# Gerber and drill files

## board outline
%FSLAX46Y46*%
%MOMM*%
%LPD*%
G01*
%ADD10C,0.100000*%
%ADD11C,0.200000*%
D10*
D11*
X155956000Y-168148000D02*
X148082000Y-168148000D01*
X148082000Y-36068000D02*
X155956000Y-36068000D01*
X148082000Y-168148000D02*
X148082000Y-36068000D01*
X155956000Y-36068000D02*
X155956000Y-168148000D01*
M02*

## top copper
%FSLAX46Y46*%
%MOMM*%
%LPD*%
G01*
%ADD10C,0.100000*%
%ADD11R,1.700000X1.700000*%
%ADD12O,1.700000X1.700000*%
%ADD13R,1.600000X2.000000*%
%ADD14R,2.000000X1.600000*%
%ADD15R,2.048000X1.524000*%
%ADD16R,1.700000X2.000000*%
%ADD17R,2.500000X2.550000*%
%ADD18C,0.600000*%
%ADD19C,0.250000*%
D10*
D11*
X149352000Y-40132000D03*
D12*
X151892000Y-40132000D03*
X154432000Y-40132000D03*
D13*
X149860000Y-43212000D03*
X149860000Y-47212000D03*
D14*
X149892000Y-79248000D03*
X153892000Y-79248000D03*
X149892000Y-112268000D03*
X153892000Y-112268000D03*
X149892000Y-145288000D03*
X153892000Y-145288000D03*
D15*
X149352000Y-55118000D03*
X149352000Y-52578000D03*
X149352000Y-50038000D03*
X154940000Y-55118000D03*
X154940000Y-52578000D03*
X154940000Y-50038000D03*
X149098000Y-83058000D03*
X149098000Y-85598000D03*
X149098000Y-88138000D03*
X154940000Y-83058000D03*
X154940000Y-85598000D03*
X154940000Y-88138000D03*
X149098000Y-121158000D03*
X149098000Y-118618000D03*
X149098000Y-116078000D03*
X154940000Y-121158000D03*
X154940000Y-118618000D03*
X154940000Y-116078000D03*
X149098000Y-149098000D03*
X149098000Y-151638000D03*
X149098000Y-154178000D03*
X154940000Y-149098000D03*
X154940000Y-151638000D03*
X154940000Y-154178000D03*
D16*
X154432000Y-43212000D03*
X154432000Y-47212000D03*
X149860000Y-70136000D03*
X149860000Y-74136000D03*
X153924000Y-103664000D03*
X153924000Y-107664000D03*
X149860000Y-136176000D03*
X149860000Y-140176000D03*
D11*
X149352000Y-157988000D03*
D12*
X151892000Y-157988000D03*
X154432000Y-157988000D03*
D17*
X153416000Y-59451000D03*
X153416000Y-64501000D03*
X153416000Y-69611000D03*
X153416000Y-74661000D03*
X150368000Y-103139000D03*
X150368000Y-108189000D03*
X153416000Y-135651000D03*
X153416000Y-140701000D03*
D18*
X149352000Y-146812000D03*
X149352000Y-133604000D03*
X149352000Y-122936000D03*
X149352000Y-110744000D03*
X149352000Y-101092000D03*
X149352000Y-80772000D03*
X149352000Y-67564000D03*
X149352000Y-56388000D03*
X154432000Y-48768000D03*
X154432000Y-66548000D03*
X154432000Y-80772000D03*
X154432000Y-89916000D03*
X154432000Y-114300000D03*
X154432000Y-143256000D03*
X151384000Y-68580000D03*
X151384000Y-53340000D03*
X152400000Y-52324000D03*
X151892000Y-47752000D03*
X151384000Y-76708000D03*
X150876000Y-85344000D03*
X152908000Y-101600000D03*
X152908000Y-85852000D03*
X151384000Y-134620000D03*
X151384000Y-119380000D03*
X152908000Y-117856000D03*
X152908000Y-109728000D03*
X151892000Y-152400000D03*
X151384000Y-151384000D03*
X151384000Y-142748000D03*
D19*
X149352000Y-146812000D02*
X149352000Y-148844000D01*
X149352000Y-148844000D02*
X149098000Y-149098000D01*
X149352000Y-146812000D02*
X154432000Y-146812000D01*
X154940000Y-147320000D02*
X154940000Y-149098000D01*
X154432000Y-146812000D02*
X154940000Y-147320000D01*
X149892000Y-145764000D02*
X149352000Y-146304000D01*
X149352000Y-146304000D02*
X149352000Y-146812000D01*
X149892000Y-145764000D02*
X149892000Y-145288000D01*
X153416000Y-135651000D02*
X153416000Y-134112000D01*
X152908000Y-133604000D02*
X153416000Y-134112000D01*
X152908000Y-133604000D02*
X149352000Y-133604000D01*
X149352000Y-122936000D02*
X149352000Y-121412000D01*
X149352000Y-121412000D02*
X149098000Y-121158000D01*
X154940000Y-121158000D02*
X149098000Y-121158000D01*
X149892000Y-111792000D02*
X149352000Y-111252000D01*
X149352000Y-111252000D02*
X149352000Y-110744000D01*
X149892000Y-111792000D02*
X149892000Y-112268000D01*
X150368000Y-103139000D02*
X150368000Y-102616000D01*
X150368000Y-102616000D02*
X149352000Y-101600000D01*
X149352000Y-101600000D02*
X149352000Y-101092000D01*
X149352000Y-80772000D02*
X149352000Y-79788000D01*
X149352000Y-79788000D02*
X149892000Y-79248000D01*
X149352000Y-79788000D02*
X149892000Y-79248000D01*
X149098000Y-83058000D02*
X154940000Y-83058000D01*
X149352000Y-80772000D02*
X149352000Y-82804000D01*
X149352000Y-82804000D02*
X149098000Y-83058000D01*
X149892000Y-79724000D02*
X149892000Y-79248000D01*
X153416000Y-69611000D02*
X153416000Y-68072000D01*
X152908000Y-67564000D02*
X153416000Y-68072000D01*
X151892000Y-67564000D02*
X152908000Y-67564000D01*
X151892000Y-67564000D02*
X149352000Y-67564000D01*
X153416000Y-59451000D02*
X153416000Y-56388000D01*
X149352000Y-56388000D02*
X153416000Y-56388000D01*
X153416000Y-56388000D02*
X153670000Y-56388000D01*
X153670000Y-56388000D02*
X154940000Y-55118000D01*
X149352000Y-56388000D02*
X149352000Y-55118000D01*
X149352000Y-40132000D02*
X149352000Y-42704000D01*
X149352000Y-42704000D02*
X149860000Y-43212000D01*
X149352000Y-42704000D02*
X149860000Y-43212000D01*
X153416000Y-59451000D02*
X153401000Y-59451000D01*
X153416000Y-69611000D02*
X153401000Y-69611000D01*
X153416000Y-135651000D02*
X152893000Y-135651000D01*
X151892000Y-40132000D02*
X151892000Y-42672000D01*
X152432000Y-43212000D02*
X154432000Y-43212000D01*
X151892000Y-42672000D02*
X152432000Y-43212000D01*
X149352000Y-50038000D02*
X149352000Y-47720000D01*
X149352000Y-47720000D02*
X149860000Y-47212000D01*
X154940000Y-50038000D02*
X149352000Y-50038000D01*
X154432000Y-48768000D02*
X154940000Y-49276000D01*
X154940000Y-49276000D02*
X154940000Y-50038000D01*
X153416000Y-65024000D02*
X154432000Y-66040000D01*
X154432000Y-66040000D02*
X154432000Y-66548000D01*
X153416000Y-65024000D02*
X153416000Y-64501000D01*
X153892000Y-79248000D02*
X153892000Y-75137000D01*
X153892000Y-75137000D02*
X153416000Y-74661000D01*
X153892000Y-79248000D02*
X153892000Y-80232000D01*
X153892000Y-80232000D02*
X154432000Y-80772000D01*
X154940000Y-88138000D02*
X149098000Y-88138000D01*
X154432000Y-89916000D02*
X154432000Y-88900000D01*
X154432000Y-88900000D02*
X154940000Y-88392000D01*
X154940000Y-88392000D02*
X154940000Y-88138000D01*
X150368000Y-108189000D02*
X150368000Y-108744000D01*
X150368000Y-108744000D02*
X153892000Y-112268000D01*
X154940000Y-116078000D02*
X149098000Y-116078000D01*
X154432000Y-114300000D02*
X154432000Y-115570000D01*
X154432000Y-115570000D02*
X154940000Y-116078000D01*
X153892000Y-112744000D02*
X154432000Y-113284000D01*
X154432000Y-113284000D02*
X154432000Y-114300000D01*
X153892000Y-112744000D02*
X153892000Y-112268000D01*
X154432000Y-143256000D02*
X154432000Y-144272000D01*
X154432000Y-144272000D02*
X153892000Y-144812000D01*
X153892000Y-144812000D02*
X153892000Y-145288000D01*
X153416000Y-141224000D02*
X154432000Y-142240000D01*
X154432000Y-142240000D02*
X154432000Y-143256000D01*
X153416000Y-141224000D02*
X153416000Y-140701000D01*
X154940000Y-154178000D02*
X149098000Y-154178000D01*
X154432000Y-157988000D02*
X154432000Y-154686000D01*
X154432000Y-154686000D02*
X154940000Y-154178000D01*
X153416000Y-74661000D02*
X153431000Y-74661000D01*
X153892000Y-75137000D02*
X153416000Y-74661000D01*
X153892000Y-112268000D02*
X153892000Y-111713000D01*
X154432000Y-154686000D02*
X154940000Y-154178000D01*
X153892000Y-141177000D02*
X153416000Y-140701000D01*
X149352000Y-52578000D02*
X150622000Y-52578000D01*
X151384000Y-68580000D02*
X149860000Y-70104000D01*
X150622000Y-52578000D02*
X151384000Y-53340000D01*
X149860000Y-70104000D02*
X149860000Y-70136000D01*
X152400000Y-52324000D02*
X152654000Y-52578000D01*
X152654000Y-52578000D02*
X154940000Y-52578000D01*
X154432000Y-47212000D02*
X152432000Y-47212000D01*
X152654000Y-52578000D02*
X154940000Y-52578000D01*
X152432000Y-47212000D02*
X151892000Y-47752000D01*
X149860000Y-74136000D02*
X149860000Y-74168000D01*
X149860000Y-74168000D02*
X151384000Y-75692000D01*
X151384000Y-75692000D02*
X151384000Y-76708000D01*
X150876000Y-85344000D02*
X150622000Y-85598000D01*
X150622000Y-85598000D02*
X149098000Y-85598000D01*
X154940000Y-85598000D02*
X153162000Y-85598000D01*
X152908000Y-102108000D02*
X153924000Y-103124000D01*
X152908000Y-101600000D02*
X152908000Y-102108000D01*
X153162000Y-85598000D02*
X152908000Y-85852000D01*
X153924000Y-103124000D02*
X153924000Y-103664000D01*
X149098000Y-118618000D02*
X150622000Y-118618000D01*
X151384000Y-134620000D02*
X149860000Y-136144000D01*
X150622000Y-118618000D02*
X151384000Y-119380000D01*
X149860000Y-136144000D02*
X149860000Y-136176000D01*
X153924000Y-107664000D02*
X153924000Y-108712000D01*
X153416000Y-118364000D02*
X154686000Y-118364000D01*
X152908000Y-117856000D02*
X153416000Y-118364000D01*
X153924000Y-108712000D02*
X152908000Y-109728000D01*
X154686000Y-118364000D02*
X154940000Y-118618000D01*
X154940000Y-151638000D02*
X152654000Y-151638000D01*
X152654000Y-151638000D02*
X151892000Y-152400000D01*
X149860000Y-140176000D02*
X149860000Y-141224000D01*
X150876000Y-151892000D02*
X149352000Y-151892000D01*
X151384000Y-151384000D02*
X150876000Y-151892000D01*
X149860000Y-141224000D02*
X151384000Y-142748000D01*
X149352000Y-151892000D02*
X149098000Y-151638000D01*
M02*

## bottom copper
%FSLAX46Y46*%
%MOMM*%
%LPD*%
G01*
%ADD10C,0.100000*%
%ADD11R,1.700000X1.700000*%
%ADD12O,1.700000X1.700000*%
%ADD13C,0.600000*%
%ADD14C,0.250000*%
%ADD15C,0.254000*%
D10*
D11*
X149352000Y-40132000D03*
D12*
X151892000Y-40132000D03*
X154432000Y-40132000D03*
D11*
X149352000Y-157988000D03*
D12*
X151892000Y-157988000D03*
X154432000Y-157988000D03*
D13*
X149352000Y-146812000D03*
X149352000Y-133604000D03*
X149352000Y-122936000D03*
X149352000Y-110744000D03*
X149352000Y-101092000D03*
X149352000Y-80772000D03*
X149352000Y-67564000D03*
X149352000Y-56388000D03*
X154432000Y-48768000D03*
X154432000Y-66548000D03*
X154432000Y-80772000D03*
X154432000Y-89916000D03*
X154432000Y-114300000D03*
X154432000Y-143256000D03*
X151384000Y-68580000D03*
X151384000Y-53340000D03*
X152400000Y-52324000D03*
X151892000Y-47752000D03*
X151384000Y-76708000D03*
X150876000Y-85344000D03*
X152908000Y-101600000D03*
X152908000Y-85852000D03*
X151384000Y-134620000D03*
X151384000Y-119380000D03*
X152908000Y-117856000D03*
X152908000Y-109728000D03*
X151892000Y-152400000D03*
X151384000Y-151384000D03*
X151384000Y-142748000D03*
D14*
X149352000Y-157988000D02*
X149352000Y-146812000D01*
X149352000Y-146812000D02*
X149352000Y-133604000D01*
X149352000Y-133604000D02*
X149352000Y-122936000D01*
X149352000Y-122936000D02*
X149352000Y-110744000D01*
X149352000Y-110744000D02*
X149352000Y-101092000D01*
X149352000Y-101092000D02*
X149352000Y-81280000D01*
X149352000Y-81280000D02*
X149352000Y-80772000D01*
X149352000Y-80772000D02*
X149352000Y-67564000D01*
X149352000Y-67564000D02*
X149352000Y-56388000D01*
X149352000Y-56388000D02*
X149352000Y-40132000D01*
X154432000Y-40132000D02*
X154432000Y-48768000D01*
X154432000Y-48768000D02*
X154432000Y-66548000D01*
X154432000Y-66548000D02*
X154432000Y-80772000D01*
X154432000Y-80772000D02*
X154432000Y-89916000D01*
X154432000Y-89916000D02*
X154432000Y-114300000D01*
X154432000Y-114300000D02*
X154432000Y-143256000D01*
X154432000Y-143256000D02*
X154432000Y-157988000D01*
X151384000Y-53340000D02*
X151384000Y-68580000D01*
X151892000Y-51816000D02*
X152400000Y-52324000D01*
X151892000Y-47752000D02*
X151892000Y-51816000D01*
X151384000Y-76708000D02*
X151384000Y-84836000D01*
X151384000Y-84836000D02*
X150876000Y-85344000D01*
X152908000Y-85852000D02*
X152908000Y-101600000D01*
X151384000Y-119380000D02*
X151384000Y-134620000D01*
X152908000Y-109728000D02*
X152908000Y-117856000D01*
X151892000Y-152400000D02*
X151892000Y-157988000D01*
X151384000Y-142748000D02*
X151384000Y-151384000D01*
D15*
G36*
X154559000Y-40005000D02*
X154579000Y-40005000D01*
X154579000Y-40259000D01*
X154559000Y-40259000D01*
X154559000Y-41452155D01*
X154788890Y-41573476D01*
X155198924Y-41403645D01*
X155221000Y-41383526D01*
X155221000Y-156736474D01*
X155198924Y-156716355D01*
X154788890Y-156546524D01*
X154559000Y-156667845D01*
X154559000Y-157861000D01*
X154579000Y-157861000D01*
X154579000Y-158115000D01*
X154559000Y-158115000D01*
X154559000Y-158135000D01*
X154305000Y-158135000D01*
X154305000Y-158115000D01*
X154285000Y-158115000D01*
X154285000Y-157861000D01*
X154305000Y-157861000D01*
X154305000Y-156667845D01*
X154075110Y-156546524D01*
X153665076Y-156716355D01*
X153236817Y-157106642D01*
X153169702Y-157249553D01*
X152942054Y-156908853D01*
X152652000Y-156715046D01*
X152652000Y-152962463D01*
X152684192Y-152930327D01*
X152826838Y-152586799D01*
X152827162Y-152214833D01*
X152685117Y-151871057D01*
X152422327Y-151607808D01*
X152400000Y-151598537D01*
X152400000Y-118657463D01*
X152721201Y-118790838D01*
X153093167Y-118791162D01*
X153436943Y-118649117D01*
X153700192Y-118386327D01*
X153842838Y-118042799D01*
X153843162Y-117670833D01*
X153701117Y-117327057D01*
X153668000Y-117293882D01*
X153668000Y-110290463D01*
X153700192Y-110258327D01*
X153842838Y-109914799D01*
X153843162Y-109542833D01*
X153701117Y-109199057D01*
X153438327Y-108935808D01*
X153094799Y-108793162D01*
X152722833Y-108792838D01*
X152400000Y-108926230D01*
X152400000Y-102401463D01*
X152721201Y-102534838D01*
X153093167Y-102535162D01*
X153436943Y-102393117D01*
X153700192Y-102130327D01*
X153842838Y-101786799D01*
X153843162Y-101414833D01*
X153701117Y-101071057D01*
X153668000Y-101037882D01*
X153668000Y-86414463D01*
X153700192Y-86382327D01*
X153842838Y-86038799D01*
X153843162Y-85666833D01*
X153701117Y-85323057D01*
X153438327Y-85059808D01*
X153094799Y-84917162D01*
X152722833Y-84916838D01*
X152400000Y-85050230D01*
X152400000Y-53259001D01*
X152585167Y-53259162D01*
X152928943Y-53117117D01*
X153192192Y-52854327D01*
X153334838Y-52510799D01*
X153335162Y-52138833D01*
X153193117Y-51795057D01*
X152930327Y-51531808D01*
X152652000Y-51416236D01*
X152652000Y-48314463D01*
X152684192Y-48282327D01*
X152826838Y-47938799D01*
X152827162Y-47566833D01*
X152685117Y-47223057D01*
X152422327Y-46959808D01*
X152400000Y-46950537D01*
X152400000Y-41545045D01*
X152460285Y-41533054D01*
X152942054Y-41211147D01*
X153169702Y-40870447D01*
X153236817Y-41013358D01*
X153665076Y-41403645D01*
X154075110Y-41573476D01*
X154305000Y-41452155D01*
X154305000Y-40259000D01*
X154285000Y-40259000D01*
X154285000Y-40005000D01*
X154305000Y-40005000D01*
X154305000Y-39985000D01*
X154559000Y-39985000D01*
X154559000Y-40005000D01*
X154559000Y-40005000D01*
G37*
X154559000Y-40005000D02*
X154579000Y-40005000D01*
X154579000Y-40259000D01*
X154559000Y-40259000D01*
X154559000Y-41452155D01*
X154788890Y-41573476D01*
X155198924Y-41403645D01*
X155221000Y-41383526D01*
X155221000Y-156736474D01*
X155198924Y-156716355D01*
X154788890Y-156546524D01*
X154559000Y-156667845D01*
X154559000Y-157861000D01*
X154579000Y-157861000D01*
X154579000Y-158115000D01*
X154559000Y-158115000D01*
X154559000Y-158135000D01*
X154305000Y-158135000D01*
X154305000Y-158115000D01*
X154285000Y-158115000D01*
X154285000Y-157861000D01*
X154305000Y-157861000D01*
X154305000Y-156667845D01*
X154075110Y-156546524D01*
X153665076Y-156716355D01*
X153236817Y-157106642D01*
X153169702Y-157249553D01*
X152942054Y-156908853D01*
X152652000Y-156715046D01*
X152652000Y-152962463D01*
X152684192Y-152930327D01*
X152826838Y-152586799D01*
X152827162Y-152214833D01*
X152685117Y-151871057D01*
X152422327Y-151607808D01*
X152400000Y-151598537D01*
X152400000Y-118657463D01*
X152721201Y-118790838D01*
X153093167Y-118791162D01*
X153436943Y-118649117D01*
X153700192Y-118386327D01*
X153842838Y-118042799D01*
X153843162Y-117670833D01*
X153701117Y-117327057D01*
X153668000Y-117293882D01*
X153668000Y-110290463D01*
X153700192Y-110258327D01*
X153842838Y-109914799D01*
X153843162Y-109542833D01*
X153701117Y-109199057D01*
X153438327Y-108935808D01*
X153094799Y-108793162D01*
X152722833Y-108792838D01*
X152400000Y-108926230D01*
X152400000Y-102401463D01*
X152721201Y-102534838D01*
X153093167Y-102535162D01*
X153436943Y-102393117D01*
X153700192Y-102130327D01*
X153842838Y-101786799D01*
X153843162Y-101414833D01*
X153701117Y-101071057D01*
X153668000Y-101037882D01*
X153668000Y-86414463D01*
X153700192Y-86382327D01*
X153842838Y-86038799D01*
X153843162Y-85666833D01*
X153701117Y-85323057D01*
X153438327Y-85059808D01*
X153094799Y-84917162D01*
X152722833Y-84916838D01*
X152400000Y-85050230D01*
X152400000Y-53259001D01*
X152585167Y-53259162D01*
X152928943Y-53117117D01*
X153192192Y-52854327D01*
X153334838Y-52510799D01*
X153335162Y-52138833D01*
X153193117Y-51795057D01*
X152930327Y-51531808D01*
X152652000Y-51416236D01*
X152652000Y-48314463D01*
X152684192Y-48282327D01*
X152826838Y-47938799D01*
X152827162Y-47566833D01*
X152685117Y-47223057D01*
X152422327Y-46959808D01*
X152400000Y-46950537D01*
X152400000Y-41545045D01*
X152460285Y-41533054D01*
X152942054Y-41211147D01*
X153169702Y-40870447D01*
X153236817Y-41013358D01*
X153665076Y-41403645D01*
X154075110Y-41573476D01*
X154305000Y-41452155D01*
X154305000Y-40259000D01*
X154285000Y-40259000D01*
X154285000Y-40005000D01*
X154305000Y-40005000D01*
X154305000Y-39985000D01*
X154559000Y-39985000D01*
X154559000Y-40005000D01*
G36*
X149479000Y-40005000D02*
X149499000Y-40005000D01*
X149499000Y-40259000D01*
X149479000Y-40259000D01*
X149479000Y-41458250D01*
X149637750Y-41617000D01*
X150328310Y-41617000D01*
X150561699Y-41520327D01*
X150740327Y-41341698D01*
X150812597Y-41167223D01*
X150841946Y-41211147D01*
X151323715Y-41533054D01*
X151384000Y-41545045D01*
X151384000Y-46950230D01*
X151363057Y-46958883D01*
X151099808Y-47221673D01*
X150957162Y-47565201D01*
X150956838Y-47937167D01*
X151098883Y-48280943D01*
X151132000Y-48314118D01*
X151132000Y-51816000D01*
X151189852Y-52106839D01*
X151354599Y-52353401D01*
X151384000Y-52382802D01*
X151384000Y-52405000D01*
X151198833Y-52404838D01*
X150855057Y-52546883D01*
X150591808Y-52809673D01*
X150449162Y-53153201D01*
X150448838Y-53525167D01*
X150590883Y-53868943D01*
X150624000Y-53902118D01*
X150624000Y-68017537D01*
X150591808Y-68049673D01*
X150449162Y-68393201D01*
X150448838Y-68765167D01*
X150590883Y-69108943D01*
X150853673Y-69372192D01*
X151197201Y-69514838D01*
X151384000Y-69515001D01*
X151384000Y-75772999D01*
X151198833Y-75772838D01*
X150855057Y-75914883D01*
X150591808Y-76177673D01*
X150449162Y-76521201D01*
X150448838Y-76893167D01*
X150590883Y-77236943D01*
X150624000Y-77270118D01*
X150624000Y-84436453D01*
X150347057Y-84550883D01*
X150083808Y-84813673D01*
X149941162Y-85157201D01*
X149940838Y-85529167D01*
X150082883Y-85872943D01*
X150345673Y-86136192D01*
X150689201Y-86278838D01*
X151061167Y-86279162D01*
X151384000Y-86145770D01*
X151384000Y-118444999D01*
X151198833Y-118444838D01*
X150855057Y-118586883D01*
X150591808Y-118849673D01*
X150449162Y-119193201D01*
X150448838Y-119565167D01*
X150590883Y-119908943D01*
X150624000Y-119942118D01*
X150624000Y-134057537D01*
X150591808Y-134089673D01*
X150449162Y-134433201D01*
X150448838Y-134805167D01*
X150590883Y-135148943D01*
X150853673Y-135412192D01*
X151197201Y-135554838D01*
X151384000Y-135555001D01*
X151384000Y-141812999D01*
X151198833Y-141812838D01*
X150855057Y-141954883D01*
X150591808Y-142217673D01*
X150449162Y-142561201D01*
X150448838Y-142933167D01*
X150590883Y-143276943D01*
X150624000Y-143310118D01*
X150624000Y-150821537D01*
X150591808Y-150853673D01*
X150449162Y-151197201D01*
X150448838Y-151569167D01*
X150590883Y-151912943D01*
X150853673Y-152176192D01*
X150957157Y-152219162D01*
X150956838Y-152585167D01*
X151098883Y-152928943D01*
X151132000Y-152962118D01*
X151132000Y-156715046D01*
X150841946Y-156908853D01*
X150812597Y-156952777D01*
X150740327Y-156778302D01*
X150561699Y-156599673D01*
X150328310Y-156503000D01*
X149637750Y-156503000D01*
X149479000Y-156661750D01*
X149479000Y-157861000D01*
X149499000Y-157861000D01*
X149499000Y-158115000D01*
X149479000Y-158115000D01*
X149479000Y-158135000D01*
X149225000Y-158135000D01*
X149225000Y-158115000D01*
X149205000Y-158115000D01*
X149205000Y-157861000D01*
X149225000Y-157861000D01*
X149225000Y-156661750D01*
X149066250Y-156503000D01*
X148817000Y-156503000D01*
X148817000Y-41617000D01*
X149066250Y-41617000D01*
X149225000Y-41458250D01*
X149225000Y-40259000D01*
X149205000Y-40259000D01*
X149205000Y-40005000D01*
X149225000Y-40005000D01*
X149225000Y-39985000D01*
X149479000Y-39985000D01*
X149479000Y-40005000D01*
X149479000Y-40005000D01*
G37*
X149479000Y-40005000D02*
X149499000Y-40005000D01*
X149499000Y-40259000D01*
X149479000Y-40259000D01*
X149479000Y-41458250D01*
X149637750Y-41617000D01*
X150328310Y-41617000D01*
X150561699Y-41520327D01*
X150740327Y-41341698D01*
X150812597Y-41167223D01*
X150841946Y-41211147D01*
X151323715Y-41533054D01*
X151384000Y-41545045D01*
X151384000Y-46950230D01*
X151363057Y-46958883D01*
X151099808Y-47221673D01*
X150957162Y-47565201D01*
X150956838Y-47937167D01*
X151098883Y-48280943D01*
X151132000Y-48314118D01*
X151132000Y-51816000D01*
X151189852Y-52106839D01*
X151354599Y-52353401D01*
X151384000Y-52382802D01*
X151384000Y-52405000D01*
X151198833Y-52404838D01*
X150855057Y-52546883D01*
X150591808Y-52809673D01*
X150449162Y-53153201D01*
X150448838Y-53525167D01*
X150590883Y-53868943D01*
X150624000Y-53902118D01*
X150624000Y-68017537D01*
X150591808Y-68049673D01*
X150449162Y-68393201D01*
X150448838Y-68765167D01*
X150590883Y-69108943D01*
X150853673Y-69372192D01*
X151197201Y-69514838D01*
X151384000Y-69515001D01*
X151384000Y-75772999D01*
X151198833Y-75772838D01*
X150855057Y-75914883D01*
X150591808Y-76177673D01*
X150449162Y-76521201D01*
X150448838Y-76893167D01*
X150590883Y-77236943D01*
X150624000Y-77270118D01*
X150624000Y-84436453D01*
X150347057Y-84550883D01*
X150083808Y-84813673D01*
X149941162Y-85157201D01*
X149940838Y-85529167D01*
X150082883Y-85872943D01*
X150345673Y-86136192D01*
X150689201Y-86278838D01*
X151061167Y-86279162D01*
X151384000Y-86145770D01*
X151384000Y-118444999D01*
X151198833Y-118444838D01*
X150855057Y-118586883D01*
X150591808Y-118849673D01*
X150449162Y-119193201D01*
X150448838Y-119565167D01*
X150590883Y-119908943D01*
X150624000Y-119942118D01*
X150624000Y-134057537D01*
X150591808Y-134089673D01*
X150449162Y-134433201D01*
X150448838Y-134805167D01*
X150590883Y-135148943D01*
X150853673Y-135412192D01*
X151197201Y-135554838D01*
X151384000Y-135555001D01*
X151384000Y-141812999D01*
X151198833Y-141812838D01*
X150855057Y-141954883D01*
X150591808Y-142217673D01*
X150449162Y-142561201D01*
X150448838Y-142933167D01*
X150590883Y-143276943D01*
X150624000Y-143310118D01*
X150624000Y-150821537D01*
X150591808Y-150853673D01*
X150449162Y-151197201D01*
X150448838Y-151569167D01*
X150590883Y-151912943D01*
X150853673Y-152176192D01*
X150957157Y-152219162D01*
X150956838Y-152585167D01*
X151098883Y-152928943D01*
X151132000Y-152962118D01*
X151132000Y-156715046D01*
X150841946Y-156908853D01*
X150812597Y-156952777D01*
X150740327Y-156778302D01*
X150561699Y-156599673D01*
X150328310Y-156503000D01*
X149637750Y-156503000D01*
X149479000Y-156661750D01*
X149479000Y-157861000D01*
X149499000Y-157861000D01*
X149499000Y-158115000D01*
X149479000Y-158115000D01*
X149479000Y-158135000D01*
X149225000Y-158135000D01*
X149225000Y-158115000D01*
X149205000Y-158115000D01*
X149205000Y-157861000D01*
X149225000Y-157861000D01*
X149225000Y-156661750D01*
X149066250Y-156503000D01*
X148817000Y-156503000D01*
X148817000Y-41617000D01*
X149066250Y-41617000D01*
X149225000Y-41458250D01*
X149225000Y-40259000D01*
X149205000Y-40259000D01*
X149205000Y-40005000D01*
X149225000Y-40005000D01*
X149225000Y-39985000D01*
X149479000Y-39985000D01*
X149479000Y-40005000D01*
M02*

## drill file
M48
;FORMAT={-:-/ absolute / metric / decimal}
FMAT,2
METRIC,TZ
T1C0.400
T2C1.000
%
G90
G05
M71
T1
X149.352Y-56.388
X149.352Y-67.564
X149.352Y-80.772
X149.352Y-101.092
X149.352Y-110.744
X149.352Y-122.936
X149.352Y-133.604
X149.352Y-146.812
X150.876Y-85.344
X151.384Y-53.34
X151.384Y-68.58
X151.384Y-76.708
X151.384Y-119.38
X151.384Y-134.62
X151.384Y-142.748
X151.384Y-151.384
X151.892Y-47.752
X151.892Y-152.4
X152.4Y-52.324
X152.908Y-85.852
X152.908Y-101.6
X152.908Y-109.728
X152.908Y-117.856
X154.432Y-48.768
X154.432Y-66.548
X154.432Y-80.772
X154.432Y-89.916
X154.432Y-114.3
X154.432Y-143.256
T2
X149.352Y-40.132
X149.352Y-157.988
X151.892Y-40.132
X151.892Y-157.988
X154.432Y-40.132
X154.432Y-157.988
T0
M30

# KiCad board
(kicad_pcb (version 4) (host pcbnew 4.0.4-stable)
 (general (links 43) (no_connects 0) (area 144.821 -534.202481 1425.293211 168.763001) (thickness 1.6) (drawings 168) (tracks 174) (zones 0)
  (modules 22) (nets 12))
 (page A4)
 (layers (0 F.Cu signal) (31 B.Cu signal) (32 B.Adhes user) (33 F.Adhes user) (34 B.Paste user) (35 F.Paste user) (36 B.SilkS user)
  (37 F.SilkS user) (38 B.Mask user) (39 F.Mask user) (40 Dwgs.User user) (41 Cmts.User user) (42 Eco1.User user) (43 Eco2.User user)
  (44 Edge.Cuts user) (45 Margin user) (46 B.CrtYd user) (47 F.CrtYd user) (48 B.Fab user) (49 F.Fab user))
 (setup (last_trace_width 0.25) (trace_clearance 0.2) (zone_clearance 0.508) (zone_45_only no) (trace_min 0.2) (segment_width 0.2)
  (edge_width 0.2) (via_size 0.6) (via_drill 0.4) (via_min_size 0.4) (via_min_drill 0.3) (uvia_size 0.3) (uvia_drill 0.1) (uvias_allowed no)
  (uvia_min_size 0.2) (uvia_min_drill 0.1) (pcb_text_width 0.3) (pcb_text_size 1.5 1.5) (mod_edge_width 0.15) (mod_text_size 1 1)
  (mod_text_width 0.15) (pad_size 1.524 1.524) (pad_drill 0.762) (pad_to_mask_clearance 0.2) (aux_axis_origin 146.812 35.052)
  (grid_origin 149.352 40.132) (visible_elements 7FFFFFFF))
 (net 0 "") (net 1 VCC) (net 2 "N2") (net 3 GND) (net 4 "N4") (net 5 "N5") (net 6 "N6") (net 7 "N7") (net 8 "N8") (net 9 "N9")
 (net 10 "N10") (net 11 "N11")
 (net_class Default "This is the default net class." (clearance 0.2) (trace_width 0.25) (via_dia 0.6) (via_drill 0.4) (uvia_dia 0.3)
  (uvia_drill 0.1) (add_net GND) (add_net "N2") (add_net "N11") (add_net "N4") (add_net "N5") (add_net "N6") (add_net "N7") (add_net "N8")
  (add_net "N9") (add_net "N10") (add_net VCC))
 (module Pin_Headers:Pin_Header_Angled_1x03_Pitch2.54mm (layer F.Cu) (at 149.352 40.132 90)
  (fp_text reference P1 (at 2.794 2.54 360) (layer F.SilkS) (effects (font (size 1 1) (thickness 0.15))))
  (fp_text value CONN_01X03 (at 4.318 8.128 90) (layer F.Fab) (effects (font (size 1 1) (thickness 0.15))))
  (pad 1 thru_hole rect (at 0 0 90) (size 1.7 1.7) (drill 1) (layers *.Cu *.Mask) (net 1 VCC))
  (pad 2 thru_hole oval (at 0 2.54 90) (size 1.7 1.7) (drill 1) (layers *.Cu *.Mask) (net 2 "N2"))
  (pad 3 thru_hole oval (at 0 5.08 90) (size 1.7 1.7) (drill 1) (layers *.Cu *.Mask) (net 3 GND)))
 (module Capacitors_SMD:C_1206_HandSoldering (layer F.Cu) (at 149.86 45.212 270)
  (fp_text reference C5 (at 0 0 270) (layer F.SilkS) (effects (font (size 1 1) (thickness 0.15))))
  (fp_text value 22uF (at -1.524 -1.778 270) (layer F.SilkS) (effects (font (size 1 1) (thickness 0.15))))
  (pad 1 smd rect (at -2 0 270) (size 2 1.6) (layers F.Cu F.Paste F.Mask) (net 1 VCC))
  (pad 2 smd rect (at 2 0 270) (size 2 1.6) (layers F.Cu F.Paste F.Mask) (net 3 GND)))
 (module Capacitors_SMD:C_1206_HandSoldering (layer F.Cu) (at 151.892 79.248)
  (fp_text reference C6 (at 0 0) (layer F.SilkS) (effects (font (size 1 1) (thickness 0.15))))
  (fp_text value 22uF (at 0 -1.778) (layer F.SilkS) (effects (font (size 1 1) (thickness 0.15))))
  (pad 1 smd rect (at -2 0) (size 2 1.6) (layers F.Cu F.Paste F.Mask) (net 1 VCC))
  (pad 2 smd rect (at 2 0) (size 2 1.6) (layers F.Cu F.Paste F.Mask) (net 3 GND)))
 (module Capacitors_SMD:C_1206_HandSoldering (layer F.Cu) (at 151.892 112.268)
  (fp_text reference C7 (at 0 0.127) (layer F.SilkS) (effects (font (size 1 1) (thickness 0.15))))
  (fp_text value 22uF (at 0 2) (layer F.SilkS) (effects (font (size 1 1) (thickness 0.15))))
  (pad 1 smd rect (at -2 0) (size 2 1.6) (layers F.Cu F.Paste F.Mask) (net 1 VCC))
  (pad 2 smd rect (at 2 0) (size 2 1.6) (layers F.Cu F.Paste F.Mask) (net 3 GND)))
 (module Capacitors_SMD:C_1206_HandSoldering (layer F.Cu) (at 151.892 145.288)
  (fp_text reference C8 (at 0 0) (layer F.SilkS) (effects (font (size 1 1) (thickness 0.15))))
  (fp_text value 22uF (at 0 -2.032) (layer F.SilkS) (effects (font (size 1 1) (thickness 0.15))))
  (pad 1 smd rect (at -2 0) (size 2 1.6) (layers F.Cu F.Paste F.Mask) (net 1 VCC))
  (pad 2 smd rect (at 2 0) (size 2 1.6) (layers F.Cu F.Paste F.Mask) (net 3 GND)))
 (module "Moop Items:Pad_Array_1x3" (layer F.Cu) (at 149.352 52.578 90)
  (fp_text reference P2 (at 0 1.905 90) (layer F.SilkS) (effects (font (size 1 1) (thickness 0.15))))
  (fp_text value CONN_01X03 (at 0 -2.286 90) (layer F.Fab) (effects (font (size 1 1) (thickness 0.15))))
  (pad 1 smd rect (at -2.54 0 90) (size 1.524 2.048) (layers F.Cu F.Paste F.Mask) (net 1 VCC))
  (pad 2 smd rect (at 0 0 90) (size 1.524 2.048) (layers F.Cu F.Paste F.Mask) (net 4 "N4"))
  (pad 3 smd rect (at 2.54 0 90) (size 1.524 2.048) (layers F.Cu F.Paste F.Mask) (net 3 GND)))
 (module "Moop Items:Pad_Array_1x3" (layer F.Cu) (at 154.94 52.578 90)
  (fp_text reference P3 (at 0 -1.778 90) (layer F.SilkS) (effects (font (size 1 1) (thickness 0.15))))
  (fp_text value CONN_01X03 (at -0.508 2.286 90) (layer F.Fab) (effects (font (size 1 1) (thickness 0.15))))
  (pad 1 smd rect (at -2.54 0 90) (size 1.524 2.048) (layers F.Cu F.Paste F.Mask) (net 1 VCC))
  (pad 2 smd rect (at 0 0 90) (size 1.524 2.048) (layers F.Cu F.Paste F.Mask) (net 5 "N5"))
  (pad 3 smd rect (at 2.54 0 90) (size 1.524 2.048) (layers F.Cu F.Paste F.Mask) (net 3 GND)))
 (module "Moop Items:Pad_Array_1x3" (layer F.Cu) (at 149.098 85.598 270)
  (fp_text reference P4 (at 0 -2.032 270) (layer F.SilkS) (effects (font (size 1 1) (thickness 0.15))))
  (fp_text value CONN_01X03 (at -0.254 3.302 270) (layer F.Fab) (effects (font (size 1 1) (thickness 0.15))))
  (pad 1 smd rect (at -2.54 0 270) (size 1.524 2.048) (layers F.Cu F.Paste F.Mask) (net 1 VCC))
  (pad 2 smd rect (at 0 0 270) (size 1.524 2.048) (layers F.Cu F.Paste F.Mask) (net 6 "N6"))
  (pad 3 smd rect (at 2.54 0 270) (size 1.524 2.048) (layers F.Cu F.Paste F.Mask) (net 3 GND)))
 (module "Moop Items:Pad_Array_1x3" (layer F.Cu) (at 154.94 85.598 270)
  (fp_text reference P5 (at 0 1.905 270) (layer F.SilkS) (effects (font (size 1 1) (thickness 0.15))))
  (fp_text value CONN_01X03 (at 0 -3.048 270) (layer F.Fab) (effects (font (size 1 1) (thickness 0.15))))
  (pad 1 smd rect (at -2.54 0 270) (size 1.524 2.048) (layers F.Cu F.Paste F.Mask) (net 1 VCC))
  (pad 2 smd rect (at 0 0 270) (size 1.524 2.048) (layers F.Cu F.Paste F.Mask) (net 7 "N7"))
  (pad 3 smd rect (at 2.54 0 270) (size 1.524 2.048) (layers F.Cu F.Paste F.Mask) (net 3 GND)))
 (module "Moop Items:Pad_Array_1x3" (layer F.Cu) (at 149.098 118.618 90)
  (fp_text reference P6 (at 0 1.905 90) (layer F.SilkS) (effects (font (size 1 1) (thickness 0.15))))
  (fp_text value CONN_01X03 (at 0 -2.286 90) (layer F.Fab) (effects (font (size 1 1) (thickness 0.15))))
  (pad 1 smd rect (at -2.54 0 90) (size 1.524 2.048) (layers F.Cu F.Paste F.Mask) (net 1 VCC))
  (pad 2 smd rect (at 0 0 90) (size 1.524 2.048) (layers F.Cu F.Paste F.Mask) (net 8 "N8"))
  (pad 3 smd rect (at 2.54 0 90) (size 1.524 2.048) (layers F.Cu F.Paste F.Mask) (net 3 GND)))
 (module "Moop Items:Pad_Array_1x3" (layer F.Cu) (at 154.94 118.618 90)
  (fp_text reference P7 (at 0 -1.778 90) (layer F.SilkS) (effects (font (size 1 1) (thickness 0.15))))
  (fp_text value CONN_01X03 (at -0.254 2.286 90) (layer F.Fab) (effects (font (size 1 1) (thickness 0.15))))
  (pad 1 smd rect (at -2.54 0 90) (size 1.524 2.048) (layers F.Cu F.Paste F.Mask) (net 1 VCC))
  (pad 2 smd rect (at 0 0 90) (size 1.524 2.048) (layers F.Cu F.Paste F.Mask) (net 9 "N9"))
  (pad 3 smd rect (at 2.54 0 90) (size 1.524 2.048) (layers F.Cu F.Paste F.Mask) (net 3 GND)))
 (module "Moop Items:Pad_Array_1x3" (layer F.Cu) (at 149.098 151.638 270)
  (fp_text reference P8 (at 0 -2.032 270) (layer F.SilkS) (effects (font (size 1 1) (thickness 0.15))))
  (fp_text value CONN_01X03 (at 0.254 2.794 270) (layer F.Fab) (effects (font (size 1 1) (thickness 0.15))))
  (pad 1 smd rect (at -2.54 0 270) (size 1.524 2.048) (layers F.Cu F.Paste F.Mask) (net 1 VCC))
  (pad 2 smd rect (at 0 0 270) (size 1.524 2.048) (layers F.Cu F.Paste F.Mask) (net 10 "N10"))
  (pad 3 smd rect (at 2.54 0 270) (size 1.524 2.048) (layers F.Cu F.Paste F.Mask) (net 3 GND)))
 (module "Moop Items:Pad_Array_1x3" (layer F.Cu) (at 154.94 151.638 270)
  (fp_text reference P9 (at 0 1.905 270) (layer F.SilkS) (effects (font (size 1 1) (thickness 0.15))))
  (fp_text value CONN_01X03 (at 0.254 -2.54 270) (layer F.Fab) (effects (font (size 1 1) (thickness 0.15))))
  (pad 1 smd rect (at -2.54 0 270) (size 1.524 2.048) (layers F.Cu F.Paste F.Mask) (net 1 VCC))
  (pad 2 smd rect (at 0 0 270) (size 1.524 2.048) (layers F.Cu F.Paste F.Mask) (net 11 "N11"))
  (pad 3 smd rect (at 2.54 0 270) (size 1.524 2.048) (layers F.Cu F.Paste F.Mask) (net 3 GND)))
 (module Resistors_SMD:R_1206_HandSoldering (layer F.Cu) (at 154.432 45.212 270)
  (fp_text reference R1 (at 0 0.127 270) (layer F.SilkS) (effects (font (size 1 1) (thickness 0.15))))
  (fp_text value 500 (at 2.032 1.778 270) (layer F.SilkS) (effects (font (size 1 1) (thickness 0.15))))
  (pad 1 smd rect (at -2 0 270) (size 2 1.7) (layers F.Cu F.Paste F.Mask) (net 2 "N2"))
  (pad 2 smd rect (at 2 0 270) (size 2 1.7) (layers F.Cu F.Paste F.Mask) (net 5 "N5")))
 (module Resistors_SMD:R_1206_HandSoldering (layer F.Cu) (at 149.86 72.136 270)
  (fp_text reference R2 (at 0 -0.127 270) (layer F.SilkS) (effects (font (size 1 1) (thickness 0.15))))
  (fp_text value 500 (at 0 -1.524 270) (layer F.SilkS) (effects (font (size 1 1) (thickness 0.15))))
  (pad 1 smd rect (at -2 0 270) (size 2 1.7) (layers F.Cu F.Paste F.Mask) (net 4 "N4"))
  (pad 2 smd rect (at 2 0 270) (size 2 1.7) (layers F.Cu F.Paste F.Mask) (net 6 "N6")))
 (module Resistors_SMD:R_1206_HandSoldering (layer F.Cu) (at 153.924 105.664 270)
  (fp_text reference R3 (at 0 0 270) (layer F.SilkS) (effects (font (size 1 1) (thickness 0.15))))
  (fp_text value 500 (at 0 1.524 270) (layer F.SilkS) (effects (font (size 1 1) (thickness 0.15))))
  (pad 1 smd rect (at -2 0 270) (size 2 1.7) (layers F.Cu F.Paste F.Mask) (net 7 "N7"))
  (pad 2 smd rect (at 2 0 270) (size 2 1.7) (layers F.Cu F.Paste F.Mask) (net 9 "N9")))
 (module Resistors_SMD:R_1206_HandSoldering (layer F.Cu) (at 149.86 138.176 270)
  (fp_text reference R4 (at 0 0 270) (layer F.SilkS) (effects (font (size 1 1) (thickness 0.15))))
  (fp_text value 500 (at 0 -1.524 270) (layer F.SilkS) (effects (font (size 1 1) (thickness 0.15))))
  (pad 1 smd rect (at -2 0 270) (size 2 1.7) (layers F.Cu F.Paste F.Mask) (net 8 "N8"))
  (pad 2 smd rect (at 2 0 270) (size 2 1.7) (layers F.Cu F.Paste F.Mask) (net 10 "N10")))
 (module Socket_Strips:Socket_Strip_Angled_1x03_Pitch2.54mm (layer F.Cu) (at 149.352 157.988 90)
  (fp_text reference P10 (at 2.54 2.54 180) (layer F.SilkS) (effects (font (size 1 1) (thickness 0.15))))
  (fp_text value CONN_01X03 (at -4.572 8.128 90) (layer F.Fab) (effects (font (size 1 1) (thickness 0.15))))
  (pad 1 thru_hole rect (at 0 0 90) (size 1.7 1.7) (drill 1) (layers *.Cu *.Mask) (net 1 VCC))
  (pad 2 thru_hole oval (at 0 2.54 90) (size 1.7 1.7) (drill 1) (layers *.Cu *.Mask) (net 11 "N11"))
  (pad 3 thru_hole oval (at 0 5.08 90) (size 1.7 1.7) (drill 1) (layers *.Cu *.Mask) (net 3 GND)))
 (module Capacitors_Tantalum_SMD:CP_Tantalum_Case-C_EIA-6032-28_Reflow (layer F.Cu) (at 153.416 61.976 270)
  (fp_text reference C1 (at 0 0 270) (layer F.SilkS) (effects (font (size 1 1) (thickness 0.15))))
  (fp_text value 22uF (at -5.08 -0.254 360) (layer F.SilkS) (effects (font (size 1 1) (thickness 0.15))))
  (pad 1 smd rect (at -2.525 0 270) (size 2.55 2.5) (layers F.Cu F.Paste F.Mask) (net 1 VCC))
  (pad 2 smd rect (at 2.525 0 270) (size 2.55 2.5) (layers F.Cu F.Paste F.Mask) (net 3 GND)))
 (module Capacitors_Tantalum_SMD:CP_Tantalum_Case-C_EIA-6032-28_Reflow (layer F.Cu) (at 153.416 72.136 270)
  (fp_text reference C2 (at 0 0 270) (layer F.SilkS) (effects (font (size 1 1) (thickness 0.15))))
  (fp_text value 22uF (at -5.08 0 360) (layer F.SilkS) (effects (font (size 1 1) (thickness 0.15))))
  (pad 1 smd rect (at -2.525 0 270) (size 2.55 2.5) (layers F.Cu F.Paste F.Mask) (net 1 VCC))
  (pad 2 smd rect (at 2.525 0 270) (size 2.55 2.5) (layers F.Cu F.Paste F.Mask) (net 3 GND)))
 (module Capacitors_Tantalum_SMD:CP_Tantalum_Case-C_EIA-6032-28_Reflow (layer F.Cu) (at 150.368 105.664 270)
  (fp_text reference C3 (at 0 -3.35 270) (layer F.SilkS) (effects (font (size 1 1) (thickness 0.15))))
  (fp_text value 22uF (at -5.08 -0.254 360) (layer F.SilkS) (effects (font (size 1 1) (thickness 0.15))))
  (pad 1 smd rect (at -2.525 0 270) (size 2.55 2.5) (layers F.Cu F.Paste F.Mask) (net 1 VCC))
  (pad 2 smd rect (at 2.525 0 270) (size 2.55 2.5) (layers F.Cu F.Paste F.Mask) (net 3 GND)))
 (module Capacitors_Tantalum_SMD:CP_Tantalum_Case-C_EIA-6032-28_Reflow (layer F.Cu) (at 153.416 138.176 270)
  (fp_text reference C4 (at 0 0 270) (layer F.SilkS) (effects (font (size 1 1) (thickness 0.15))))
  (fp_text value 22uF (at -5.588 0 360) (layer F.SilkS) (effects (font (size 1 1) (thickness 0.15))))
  (pad 1 smd rect (at -2.525 0 270) (size 2.55 2.5) (layers F.Cu F.Paste F.Mask) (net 1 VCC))
  (pad 2 smd rect (at 2.525 0 270) (size 2.55 2.5) (layers F.Cu F.Paste F.Mask) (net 3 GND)))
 (gr_line (start 155.956 168.148) (end 148.082 168.148) (angle 90) (layer Edge.Cuts) (width 0.2))
 (gr_line (start 148.082 36.068) (end 155.956 36.068) (angle 90) (layer Edge.Cuts) (width 0.2))
 (gr_line (start 148.082 168.148) (end 148.082 36.068) (angle 90) (layer Edge.Cuts) (width 0.2))
 (gr_line (start 155.956 36.068) (end 155.956 168.148) (angle 90) (layer Edge.Cuts) (width 0.2))
 (segment (start 149.352 146.812) (end 149.352 148.844) (width 0.25) (layer F.Cu) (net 1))
 (segment (start 149.352 148.844) (end 149.098 149.098) (width 0.25) (layer F.Cu) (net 1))
 (segment (start 149.352 146.812) (end 154.432 146.812) (width 0.25) (layer F.Cu) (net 1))
 (segment (start 154.94 147.32) (end 154.94 149.098) (width 0.25) (layer F.Cu) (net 1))
 (segment (start 154.432 146.812) (end 154.94 147.32) (width 0.25) (layer F.Cu) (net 1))
 (via (at 149.352 146.812) (size 0.6) (drill 0.4) (layers F.Cu B.Cu) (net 1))
 (segment (start 149.892 145.764) (end 149.352 146.304) (width 0.25) (layer F.Cu) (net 1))
 (segment (start 149.352 146.304) (end 149.352 146.812) (width 0.25) (layer F.Cu) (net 1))
 (segment (start 149.892 145.764) (end 149.892 145.288) (width 0.25) (layer F.Cu) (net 1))
 (via (at 149.352 133.604) (size 0.6) (drill 0.4) (layers F.Cu B.Cu) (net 1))
 (segment (start 153.416 135.651) (end 153.416 134.112) (width 0.25) (layer F.Cu) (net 1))
 (segment (start 152.908 133.604) (end 153.416 134.112) (width 0.25) (layer F.Cu) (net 1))
 (segment (start 152.908 133.604) (end 149.352 133.604) (width 0.25) (layer F.Cu) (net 1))
 (segment (start 149.352 122.936) (end 149.352 121.412) (width 0.25) (layer F.Cu) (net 1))
 (segment (start 149.352 121.412) (end 149.098 121.158) (width 0.25) (layer F.Cu) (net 1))
 (segment (start 154.94 121.158) (end 149.098 121.158) (width 0.25) (layer F.Cu) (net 1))
 (via (at 149.352 122.936) (size 0.6) (drill 0.4) (layers F.Cu B.Cu) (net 1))
 (via (at 149.352 110.744) (size 0.6) (drill 0.4) (layers F.Cu B.Cu) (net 1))
 (segment (start 149.892 111.792) (end 149.352 111.252) (width 0.25) (layer F.Cu) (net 1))
 (segment (start 149.352 111.252) (end 149.352 110.744) (width 0.25) (layer F.Cu) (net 1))
 (segment (start 149.892 111.792) (end 149.892 112.268) (width 0.25) (layer F.Cu) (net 1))
 (segment (start 150.368 103.139) (end 150.368 102.616) (width 0.25) (layer F.Cu) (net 1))
 (segment (start 150.368 102.616) (end 149.352 101.6) (width 0.25) (layer F.Cu) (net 1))
 (segment (start 149.352 101.6) (end 149.352 101.092) (width 0.25) (layer F.Cu) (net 1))
 (via (at 149.352 101.092) (size 0.6) (drill 0.4) (layers F.Cu B.Cu) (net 1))
 (segment (start 149.352 80.772) (end 149.352 79.788) (width 0.25) (layer F.Cu) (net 1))
 (segment (start 149.352 79.788) (end 149.892 79.248) (width 0.25) (layer F.Cu) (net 1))
 (segment (start 149.352 79.788) (end 149.892 79.248) (width 0.25) (layer F.Cu) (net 1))
 (segment (start 149.098 83.058) (end 154.94 83.058) (width 0.25) (layer F.Cu) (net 1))
 (segment (start 149.352 80.772) (end 149.352 82.804) (width 0.25) (layer F.Cu) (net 1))
 (segment (start 149.352 82.804) (end 149.098 83.058) (width 0.25) (layer F.Cu) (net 1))
 (via (at 149.352 80.772) (size 0.6) (drill 0.4) (layers F.Cu B.Cu) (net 1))
 (segment (start 149.892 79.724) (end 149.892 79.248) (width 0.25) (layer F.Cu) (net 1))
 (via (at 149.352 67.564) (size 0.6) (drill 0.4) (layers F.Cu B.Cu) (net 1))
 (segment (start 153.416 69.611) (end 153.416 68.072) (width 0.25) (layer F.Cu) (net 1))
 (segment (start 152.908 67.564) (end 153.416 68.072) (width 0.25) (layer F.Cu) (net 1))
 (segment (start 151.892 67.564) (end 152.908 67.564) (width 0.25) (layer F.Cu) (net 1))
 (segment (start 151.892 67.564) (end 149.352 67.564) (width 0.25) (layer F.Cu) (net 1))
 (segment (start 153.416 59.451) (end 153.416 56.388) (width 0.25) (layer F.Cu) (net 1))
 (segment (start 149.352 56.388) (end 153.416 56.388) (width 0.25) (layer F.Cu) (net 1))
 (segment (start 153.416 56.388) (end 153.67 56.388) (width 0.25) (layer F.Cu) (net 1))
 (segment (start 153.67 56.388) (end 154.94 55.118) (width 0.25) (layer F.Cu) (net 1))
 (via (at 149.352 56.388) (size 0.6) (drill 0.4) (layers F.Cu B.Cu) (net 1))
 (segment (start 149.352 56.388) (end 149.352 55.118) (width 0.25) (layer F.Cu) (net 1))
 (segment (start 149.352 40.132) (end 149.352 42.704) (width 0.25) (layer F.Cu) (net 1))
 (segment (start 149.352 42.704) (end 149.86 43.212) (width 0.25) (layer F.Cu) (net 1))
 (segment (start 149.352 157.988) (end 149.352 146.812) (width 0.25) (layer B.Cu) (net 1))
 (segment (start 149.352 146.812) (end 149.352 133.604) (width 0.25) (layer B.Cu) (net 1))
 (segment (start 149.352 133.604) (end 149.352 122.936) (width 0.25) (layer B.Cu) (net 1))
 (segment (start 149.352 122.936) (end 149.352 110.744) (width 0.25) (layer B.Cu) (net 1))
 (segment (start 149.352 110.744) (end 149.352 101.092) (width 0.25) (layer B.Cu) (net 1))
 (segment (start 149.352 101.092) (end 149.352 81.28) (width 0.25) (layer B.Cu) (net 1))
 (segment (start 149.352 81.28) (end 149.352 80.772) (width 0.25) (layer B.Cu) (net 1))
 (segment (start 149.352 80.772) (end 149.352 67.564) (width 0.25) (layer B.Cu) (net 1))
 (segment (start 149.352 67.564) (end 149.352 56.388) (width 0.25) (layer B.Cu) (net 1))
 (segment (start 149.352 56.388) (end 149.352 40.132) (width 0.25) (layer B.Cu) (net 1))
 (segment (start 149.352 42.704) (end 149.86 43.212) (width 0.25) (layer F.Cu) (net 1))
 (segment (start 153.416 59.451) (end 153.401 59.451) (width 0.25) (layer F.Cu) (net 1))
 (segment (start 153.416 69.611) (end 153.401 69.611) (width 0.25) (layer F.Cu) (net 1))
 (segment (start 153.416 135.651) (end 152.893 135.651) (width 0.25) (layer F.Cu) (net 1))
 (segment (start 151.892 40.132) (end 151.892 42.672) (width 0.25) (layer F.Cu) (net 2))
 (segment (start 152.432 43.212) (end 154.432 43.212) (width 0.25) (layer F.Cu) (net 2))
 (segment (start 151.892 42.672) (end 152.432 43.212) (width 0.25) (layer F.Cu) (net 2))
 (segment (start 149.352 50.038) (end 149.352 47.72) (width 0.25) (layer F.Cu) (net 3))
 (segment (start 149.352 47.72) (end 149.86 47.212) (width 0.25) (layer F.Cu) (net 3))
 (segment (start 154.94 50.038) (end 149.352 50.038) (width 0.25) (layer F.Cu) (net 3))
 (via (at 154.432 48.768) (size 0.6) (drill 0.4) (layers F.Cu B.Cu) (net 3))
 (segment (start 154.432 48.768) (end 154.94 49.276) (width 0.25) (layer F.Cu) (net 3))
 (segment (start 154.94 49.276) (end 154.94 50.038) (width 0.25) (layer F.Cu) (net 3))
 (via (at 154.432 66.548) (size 0.6) (drill 0.4) (layers F.Cu B.Cu) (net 3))
 (segment (start 153.416 65.024) (end 154.432 66.04) (width 0.25) (layer F.Cu) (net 3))
 (segment (start 154.432 66.04) (end 154.432 66.548) (width 0.25) (layer F.Cu) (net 3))
 (segment (start 153.416 65.024) (end 153.416 64.501) (width 0.25) (layer F.Cu) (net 3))
 (segment (start 153.892 79.248) (end 153.892 75.137) (width 0.25) (layer F.Cu) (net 3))
 (segment (start 153.892 75.137) (end 153.416 74.661) (width 0.25) (layer F.Cu) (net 3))
 (via (at 154.432 80.772) (size 0.6) (drill 0.4) (layers F.Cu B.Cu) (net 3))
 (segment (start 153.892 79.248) (end 153.892 80.232) (width 0.25) (layer F.Cu) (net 3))
 (segment (start 153.892 80.232) (end 154.432 80.772) (width 0.25) (layer F.Cu) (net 3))
 (segment (start 154.94 88.138) (end 149.098 88.138) (width 0.25) (layer F.Cu) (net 3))
 (via (at 154.432 89.916) (size 0.6) (drill 0.4) (layers F.Cu B.Cu) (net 3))
 (segment (start 154.432 89.916) (end 154.432 88.9) (width 0.25) (layer F.Cu) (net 3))
 (segment (start 154.432 88.9) (end 154.94 88.392) (width 0.25) (layer F.Cu) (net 3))
 (segment (start 154.94 88.392) (end 154.94 88.138) (width 0.25) (layer F.Cu) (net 3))
 (segment (start 150.368 108.189) (end 150.368 108.744) (width 0.25) (layer F.Cu) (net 3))
 (segment (start 150.368 108.744) (end 153.892 112.268) (width 0.25) (layer F.Cu) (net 3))
 (segment (start 154.94 116.078) (end 149.098 116.078) (width 0.25) (layer F.Cu) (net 3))
 (segment (start 154.432 114.3) (end 154.432 115.57) (width 0.25) (layer F.Cu) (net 3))
 (segment (start 154.432 115.57) (end 154.94 116.078) (width 0.25) (layer F.Cu) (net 3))
 (via (at 154.432 114.3) (size 0.6) (drill 0.4) (layers F.Cu B.Cu) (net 3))
 (segment (start 153.892 112.744) (end 154.432 113.284) (width 0.25) (layer F.Cu) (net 3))
 (segment (start 154.432 113.284) (end 154.432 114.3) (width 0.25) (layer F.Cu) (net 3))
 (segment (start 153.892 112.744) (end 153.892 112.268) (width 0.25) (layer F.Cu) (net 3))
 (segment (start 154.432 143.256) (end 154.432 144.272) (width 0.25) (layer F.Cu) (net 3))
 (segment (start 154.432 144.272) (end 153.892 144.812) (width 0.25) (layer F.Cu) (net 3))
 (segment (start 153.892 144.812) (end 153.892 145.288) (width 0.25) (layer F.Cu) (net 3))
 (via (at 154.432 143.256) (size 0.6) (drill 0.4) (layers F.Cu B.Cu) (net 3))
 (segment (start 153.416 141.224) (end 154.432 142.24) (width 0.25) (layer F.Cu) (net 3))
 (segment (start 154.432 142.24) (end 154.432 143.256) (width 0.25) (layer F.Cu) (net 3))
 (segment (start 153.416 141.224) (end 153.416 140.701) (width 0.25) (layer F.Cu) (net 3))
 (segment (start 154.94 154.178) (end 149.098 154.178) (width 0.25) (layer F.Cu) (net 3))
 (segment (start 154.432 157.988) (end 154.432 154.686) (width 0.25) (layer F.Cu) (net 3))
 (segment (start 154.432 154.686) (end 154.94 154.178) (width 0.25) (layer F.Cu) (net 3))
 (segment (start 154.432 40.132) (end 154.432 48.768) (width 0.25) (layer B.Cu) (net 3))
 (segment (start 154.432 48.768) (end 154.432 66.548) (width 0.25) (layer B.Cu) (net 3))
 (segment (start 154.432 66.548) (end 154.432 80.772) (width 0.25) (layer B.Cu) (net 3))
 (segment (start 154.432 80.772) (end 154.432 89.916) (width 0.25) (layer B.Cu) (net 3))
 (segment (start 154.432 89.916) (end 154.432 114.3) (width 0.25) (layer B.Cu) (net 3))
 (segment (start 154.432 114.3) (end 154.432 143.256) (width 0.25) (layer B.Cu) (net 3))
 (segment (start 154.432 143.256) (end 154.432 157.988) (width 0.25) (layer B.Cu) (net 3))
 (segment (start 153.416 74.661) (end 153.431 74.661) (width 0.25) (layer F.Cu) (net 3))
 (segment (start 153.892 75.137) (end 153.416 74.661) (width 0.25) (layer F.Cu) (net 3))
 (segment (start 153.892 112.268) (end 153.892 111.713) (width 0.25) (layer F.Cu) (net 3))
 (segment (start 154.432 154.686) (end 154.94 154.178) (width 0.25) (layer F.Cu) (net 3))
 (segment (start 153.892 141.177) (end 153.416 140.701) (width 0.25) (layer F.Cu) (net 3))
 (segment (start 149.352 52.578) (end 150.622 52.578) (width 0.25) (layer F.Cu) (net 4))
 (segment (start 151.384 68.58) (end 149.86 70.104) (width 0.25) (layer F.Cu) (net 4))
 (via (at 151.384 68.58) (size 0.6) (drill 0.4) (layers F.Cu B.Cu) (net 4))
 (segment (start 151.384 53.34) (end 151.384 68.58) (width 0.25) (layer B.Cu) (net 4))
 (via (at 151.384 53.34) (size 0.6) (drill 0.4) (layers F.Cu B.Cu) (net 4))
 (segment (start 150.622 52.578) (end 151.384 53.34) (width 0.25) (layer F.Cu) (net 4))
 (segment (start 149.86 70.104) (end 149.86 70.136) (width 0.25) (layer F.Cu) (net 4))
 (segment (start 151.892 51.816) (end 152.4 52.324) (width 0.25) (layer B.Cu) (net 5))
 (segment (start 152.4 52.324) (end 152.654 52.578) (width 0.25) (layer F.Cu) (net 5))
 (via (at 152.4 52.324) (size 0.6) (drill 0.4) (layers F.Cu B.Cu) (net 5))
 (segment (start 152.654 52.578) (end 154.94 52.578) (width 0.25) (layer F.Cu) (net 5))
 (segment (start 154.432 47.212) (end 152.432 47.212) (width 0.25) (layer F.Cu) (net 5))
 (segment (start 152.654 52.578) (end 154.94 52.578) (width 0.25) (layer F.Cu) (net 5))
 (segment (start 151.892 47.752) (end 151.892 51.816) (width 0.25) (layer B.Cu) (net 5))
 (via (at 151.892 47.752) (size 0.6) (drill 0.4) (layers F.Cu B.Cu) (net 5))
 (segment (start 152.432 47.212) (end 151.892 47.752) (width 0.25) (layer F.Cu) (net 5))
 (segment (start 149.86 74.136) (end 149.86 74.168) (width 0.25) (layer F.Cu) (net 6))
 (segment (start 149.86 74.168) (end 151.384 75.692) (width 0.25) (layer F.Cu) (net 6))
 (segment (start 151.384 75.692) (end 151.384 76.708) (width 0.25) (layer F.Cu) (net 6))
 (via (at 151.384 76.708) (size 0.6) (drill 0.4) (layers F.Cu B.Cu) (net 6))
 (segment (start 151.384 76.708) (end 151.384 84.836) (width 0.25) (layer B.Cu) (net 6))
 (segment (start 151.384 84.836) (end 150.876 85.344) (width 0.25) (layer B.Cu) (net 6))
 (via (at 150.876 85.344) (size 0.6) (drill 0.4) (layers F.Cu B.Cu) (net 6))
 (segment (start 150.876 85.344) (end 150.622 85.598) (width 0.25) (layer F.Cu) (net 6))
 (segment (start 150.622 85.598) (end 149.098 85.598) (width 0.25) (layer F.Cu) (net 6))
 (segment (start 154.94 85.598) (end 153.162 85.598) (width 0.25) (layer F.Cu) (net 7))
 (segment (start 152.908 102.108) (end 153.924 103.124) (width 0.25) (layer F.Cu) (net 7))
 (segment (start 152.908 101.6) (end 152.908 102.108) (width 0.25) (layer F.Cu) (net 7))
 (via (at 152.908 101.6) (size 0.6) (drill 0.4) (layers F.Cu B.Cu) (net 7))
 (segment (start 152.908 85.852) (end 152.908 101.6) (width 0.25) (layer B.Cu) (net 7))
 (via (at 152.908 85.852) (size 0.6) (drill 0.4) (layers F.Cu B.Cu) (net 7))
 (segment (start 153.162 85.598) (end 152.908 85.852) (width 0.25) (layer F.Cu) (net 7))
 (segment (start 153.924 103.124) (end 153.924 103.664) (width 0.25) (layer F.Cu) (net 7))
 (segment (start 149.098 118.618) (end 150.622 118.618) (width 0.25) (layer F.Cu) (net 8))
 (segment (start 151.384 134.62) (end 149.86 136.144) (width 0.25) (layer F.Cu) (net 8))
 (via (at 151.384 134.62) (size 0.6) (drill 0.4) (layers F.Cu B.Cu) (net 8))
 (segment (start 151.384 119.38) (end 151.384 134.62) (width 0.25) (layer B.Cu) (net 8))
 (via (at 151.384 119.38) (size 0.6) (drill 0.4) (layers F.Cu B.Cu) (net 8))
 (segment (start 150.622 118.618) (end 151.384 119.38) (width 0.25) (layer F.Cu) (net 8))
 (segment (start 149.86 136.144) (end 149.86 136.176) (width 0.25) (layer F.Cu) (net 8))
 (segment (start 153.924 107.664) (end 153.924 108.712) (width 0.25) (layer F.Cu) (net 9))
 (segment (start 153.416 118.364) (end 154.686 118.364) (width 0.25) (layer F.Cu) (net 9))
 (segment (start 152.908 117.856) (end 153.416 118.364) (width 0.25) (layer F.Cu) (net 9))
 (via (at 152.908 117.856) (size 0.6) (drill 0.4) (layers F.Cu B.Cu) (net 9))
 (segment (start 152.908 109.728) (end 152.908 117.856) (width 0.25) (layer B.Cu) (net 9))
 (via (at 152.908 109.728) (size 0.6) (drill 0.4) (layers F.Cu B.Cu) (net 9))
 (segment (start 153.924 108.712) (end 152.908 109.728) (width 0.25) (layer F.Cu) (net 9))
 (segment (start 154.686 118.364) (end 154.94 118.618) (width 0.25) (layer F.Cu) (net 9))
 (segment (start 154.94 151.638) (end 152.654 151.638) (width 0.25) (layer F.Cu) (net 11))
 (segment (start 151.892 152.4) (end 151.892 157.988) (width 0.25) (layer B.Cu) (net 11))
 (via (at 151.892 152.4) (size 0.6) (drill 0.4) (layers F.Cu B.Cu) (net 11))
 (segment (start 152.654 151.638) (end 151.892 152.4) (width 0.25) (layer F.Cu) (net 11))
 (segment (start 149.86 140.176) (end 149.86 141.224) (width 0.25) (layer F.Cu) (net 10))
 (segment (start 150.876 151.892) (end 149.352 151.892) (width 0.25) (layer F.Cu) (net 10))
 (segment (start 151.384 151.384) (end 150.876 151.892) (width 0.25) (layer F.Cu) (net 10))
 (via (at 151.384 151.384) (size 0.6) (drill 0.4) (layers F.Cu B.Cu) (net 10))
 (segment (start 151.384 142.748) (end 151.384 151.384) (width 0.25) (layer B.Cu) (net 10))
 (via (at 151.384 142.748) (size 0.6) (drill 0.4) (layers F.Cu B.Cu) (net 10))
 (segment (start 149.86 141.224) (end 151.384 142.748) (width 0.25) (layer F.Cu) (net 10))
 (segment (start 149.352 151.892) (end 149.098 151.638) (width 0.25) (layer F.Cu) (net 10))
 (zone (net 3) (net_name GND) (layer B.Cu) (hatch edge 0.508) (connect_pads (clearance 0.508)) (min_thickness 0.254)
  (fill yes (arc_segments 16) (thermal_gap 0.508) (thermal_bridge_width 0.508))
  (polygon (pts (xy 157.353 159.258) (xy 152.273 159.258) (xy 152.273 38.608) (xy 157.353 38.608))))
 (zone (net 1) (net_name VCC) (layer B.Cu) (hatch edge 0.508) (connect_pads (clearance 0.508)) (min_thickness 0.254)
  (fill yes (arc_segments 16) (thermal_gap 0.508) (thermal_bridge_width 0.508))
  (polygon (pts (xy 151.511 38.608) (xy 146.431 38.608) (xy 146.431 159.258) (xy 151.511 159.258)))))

